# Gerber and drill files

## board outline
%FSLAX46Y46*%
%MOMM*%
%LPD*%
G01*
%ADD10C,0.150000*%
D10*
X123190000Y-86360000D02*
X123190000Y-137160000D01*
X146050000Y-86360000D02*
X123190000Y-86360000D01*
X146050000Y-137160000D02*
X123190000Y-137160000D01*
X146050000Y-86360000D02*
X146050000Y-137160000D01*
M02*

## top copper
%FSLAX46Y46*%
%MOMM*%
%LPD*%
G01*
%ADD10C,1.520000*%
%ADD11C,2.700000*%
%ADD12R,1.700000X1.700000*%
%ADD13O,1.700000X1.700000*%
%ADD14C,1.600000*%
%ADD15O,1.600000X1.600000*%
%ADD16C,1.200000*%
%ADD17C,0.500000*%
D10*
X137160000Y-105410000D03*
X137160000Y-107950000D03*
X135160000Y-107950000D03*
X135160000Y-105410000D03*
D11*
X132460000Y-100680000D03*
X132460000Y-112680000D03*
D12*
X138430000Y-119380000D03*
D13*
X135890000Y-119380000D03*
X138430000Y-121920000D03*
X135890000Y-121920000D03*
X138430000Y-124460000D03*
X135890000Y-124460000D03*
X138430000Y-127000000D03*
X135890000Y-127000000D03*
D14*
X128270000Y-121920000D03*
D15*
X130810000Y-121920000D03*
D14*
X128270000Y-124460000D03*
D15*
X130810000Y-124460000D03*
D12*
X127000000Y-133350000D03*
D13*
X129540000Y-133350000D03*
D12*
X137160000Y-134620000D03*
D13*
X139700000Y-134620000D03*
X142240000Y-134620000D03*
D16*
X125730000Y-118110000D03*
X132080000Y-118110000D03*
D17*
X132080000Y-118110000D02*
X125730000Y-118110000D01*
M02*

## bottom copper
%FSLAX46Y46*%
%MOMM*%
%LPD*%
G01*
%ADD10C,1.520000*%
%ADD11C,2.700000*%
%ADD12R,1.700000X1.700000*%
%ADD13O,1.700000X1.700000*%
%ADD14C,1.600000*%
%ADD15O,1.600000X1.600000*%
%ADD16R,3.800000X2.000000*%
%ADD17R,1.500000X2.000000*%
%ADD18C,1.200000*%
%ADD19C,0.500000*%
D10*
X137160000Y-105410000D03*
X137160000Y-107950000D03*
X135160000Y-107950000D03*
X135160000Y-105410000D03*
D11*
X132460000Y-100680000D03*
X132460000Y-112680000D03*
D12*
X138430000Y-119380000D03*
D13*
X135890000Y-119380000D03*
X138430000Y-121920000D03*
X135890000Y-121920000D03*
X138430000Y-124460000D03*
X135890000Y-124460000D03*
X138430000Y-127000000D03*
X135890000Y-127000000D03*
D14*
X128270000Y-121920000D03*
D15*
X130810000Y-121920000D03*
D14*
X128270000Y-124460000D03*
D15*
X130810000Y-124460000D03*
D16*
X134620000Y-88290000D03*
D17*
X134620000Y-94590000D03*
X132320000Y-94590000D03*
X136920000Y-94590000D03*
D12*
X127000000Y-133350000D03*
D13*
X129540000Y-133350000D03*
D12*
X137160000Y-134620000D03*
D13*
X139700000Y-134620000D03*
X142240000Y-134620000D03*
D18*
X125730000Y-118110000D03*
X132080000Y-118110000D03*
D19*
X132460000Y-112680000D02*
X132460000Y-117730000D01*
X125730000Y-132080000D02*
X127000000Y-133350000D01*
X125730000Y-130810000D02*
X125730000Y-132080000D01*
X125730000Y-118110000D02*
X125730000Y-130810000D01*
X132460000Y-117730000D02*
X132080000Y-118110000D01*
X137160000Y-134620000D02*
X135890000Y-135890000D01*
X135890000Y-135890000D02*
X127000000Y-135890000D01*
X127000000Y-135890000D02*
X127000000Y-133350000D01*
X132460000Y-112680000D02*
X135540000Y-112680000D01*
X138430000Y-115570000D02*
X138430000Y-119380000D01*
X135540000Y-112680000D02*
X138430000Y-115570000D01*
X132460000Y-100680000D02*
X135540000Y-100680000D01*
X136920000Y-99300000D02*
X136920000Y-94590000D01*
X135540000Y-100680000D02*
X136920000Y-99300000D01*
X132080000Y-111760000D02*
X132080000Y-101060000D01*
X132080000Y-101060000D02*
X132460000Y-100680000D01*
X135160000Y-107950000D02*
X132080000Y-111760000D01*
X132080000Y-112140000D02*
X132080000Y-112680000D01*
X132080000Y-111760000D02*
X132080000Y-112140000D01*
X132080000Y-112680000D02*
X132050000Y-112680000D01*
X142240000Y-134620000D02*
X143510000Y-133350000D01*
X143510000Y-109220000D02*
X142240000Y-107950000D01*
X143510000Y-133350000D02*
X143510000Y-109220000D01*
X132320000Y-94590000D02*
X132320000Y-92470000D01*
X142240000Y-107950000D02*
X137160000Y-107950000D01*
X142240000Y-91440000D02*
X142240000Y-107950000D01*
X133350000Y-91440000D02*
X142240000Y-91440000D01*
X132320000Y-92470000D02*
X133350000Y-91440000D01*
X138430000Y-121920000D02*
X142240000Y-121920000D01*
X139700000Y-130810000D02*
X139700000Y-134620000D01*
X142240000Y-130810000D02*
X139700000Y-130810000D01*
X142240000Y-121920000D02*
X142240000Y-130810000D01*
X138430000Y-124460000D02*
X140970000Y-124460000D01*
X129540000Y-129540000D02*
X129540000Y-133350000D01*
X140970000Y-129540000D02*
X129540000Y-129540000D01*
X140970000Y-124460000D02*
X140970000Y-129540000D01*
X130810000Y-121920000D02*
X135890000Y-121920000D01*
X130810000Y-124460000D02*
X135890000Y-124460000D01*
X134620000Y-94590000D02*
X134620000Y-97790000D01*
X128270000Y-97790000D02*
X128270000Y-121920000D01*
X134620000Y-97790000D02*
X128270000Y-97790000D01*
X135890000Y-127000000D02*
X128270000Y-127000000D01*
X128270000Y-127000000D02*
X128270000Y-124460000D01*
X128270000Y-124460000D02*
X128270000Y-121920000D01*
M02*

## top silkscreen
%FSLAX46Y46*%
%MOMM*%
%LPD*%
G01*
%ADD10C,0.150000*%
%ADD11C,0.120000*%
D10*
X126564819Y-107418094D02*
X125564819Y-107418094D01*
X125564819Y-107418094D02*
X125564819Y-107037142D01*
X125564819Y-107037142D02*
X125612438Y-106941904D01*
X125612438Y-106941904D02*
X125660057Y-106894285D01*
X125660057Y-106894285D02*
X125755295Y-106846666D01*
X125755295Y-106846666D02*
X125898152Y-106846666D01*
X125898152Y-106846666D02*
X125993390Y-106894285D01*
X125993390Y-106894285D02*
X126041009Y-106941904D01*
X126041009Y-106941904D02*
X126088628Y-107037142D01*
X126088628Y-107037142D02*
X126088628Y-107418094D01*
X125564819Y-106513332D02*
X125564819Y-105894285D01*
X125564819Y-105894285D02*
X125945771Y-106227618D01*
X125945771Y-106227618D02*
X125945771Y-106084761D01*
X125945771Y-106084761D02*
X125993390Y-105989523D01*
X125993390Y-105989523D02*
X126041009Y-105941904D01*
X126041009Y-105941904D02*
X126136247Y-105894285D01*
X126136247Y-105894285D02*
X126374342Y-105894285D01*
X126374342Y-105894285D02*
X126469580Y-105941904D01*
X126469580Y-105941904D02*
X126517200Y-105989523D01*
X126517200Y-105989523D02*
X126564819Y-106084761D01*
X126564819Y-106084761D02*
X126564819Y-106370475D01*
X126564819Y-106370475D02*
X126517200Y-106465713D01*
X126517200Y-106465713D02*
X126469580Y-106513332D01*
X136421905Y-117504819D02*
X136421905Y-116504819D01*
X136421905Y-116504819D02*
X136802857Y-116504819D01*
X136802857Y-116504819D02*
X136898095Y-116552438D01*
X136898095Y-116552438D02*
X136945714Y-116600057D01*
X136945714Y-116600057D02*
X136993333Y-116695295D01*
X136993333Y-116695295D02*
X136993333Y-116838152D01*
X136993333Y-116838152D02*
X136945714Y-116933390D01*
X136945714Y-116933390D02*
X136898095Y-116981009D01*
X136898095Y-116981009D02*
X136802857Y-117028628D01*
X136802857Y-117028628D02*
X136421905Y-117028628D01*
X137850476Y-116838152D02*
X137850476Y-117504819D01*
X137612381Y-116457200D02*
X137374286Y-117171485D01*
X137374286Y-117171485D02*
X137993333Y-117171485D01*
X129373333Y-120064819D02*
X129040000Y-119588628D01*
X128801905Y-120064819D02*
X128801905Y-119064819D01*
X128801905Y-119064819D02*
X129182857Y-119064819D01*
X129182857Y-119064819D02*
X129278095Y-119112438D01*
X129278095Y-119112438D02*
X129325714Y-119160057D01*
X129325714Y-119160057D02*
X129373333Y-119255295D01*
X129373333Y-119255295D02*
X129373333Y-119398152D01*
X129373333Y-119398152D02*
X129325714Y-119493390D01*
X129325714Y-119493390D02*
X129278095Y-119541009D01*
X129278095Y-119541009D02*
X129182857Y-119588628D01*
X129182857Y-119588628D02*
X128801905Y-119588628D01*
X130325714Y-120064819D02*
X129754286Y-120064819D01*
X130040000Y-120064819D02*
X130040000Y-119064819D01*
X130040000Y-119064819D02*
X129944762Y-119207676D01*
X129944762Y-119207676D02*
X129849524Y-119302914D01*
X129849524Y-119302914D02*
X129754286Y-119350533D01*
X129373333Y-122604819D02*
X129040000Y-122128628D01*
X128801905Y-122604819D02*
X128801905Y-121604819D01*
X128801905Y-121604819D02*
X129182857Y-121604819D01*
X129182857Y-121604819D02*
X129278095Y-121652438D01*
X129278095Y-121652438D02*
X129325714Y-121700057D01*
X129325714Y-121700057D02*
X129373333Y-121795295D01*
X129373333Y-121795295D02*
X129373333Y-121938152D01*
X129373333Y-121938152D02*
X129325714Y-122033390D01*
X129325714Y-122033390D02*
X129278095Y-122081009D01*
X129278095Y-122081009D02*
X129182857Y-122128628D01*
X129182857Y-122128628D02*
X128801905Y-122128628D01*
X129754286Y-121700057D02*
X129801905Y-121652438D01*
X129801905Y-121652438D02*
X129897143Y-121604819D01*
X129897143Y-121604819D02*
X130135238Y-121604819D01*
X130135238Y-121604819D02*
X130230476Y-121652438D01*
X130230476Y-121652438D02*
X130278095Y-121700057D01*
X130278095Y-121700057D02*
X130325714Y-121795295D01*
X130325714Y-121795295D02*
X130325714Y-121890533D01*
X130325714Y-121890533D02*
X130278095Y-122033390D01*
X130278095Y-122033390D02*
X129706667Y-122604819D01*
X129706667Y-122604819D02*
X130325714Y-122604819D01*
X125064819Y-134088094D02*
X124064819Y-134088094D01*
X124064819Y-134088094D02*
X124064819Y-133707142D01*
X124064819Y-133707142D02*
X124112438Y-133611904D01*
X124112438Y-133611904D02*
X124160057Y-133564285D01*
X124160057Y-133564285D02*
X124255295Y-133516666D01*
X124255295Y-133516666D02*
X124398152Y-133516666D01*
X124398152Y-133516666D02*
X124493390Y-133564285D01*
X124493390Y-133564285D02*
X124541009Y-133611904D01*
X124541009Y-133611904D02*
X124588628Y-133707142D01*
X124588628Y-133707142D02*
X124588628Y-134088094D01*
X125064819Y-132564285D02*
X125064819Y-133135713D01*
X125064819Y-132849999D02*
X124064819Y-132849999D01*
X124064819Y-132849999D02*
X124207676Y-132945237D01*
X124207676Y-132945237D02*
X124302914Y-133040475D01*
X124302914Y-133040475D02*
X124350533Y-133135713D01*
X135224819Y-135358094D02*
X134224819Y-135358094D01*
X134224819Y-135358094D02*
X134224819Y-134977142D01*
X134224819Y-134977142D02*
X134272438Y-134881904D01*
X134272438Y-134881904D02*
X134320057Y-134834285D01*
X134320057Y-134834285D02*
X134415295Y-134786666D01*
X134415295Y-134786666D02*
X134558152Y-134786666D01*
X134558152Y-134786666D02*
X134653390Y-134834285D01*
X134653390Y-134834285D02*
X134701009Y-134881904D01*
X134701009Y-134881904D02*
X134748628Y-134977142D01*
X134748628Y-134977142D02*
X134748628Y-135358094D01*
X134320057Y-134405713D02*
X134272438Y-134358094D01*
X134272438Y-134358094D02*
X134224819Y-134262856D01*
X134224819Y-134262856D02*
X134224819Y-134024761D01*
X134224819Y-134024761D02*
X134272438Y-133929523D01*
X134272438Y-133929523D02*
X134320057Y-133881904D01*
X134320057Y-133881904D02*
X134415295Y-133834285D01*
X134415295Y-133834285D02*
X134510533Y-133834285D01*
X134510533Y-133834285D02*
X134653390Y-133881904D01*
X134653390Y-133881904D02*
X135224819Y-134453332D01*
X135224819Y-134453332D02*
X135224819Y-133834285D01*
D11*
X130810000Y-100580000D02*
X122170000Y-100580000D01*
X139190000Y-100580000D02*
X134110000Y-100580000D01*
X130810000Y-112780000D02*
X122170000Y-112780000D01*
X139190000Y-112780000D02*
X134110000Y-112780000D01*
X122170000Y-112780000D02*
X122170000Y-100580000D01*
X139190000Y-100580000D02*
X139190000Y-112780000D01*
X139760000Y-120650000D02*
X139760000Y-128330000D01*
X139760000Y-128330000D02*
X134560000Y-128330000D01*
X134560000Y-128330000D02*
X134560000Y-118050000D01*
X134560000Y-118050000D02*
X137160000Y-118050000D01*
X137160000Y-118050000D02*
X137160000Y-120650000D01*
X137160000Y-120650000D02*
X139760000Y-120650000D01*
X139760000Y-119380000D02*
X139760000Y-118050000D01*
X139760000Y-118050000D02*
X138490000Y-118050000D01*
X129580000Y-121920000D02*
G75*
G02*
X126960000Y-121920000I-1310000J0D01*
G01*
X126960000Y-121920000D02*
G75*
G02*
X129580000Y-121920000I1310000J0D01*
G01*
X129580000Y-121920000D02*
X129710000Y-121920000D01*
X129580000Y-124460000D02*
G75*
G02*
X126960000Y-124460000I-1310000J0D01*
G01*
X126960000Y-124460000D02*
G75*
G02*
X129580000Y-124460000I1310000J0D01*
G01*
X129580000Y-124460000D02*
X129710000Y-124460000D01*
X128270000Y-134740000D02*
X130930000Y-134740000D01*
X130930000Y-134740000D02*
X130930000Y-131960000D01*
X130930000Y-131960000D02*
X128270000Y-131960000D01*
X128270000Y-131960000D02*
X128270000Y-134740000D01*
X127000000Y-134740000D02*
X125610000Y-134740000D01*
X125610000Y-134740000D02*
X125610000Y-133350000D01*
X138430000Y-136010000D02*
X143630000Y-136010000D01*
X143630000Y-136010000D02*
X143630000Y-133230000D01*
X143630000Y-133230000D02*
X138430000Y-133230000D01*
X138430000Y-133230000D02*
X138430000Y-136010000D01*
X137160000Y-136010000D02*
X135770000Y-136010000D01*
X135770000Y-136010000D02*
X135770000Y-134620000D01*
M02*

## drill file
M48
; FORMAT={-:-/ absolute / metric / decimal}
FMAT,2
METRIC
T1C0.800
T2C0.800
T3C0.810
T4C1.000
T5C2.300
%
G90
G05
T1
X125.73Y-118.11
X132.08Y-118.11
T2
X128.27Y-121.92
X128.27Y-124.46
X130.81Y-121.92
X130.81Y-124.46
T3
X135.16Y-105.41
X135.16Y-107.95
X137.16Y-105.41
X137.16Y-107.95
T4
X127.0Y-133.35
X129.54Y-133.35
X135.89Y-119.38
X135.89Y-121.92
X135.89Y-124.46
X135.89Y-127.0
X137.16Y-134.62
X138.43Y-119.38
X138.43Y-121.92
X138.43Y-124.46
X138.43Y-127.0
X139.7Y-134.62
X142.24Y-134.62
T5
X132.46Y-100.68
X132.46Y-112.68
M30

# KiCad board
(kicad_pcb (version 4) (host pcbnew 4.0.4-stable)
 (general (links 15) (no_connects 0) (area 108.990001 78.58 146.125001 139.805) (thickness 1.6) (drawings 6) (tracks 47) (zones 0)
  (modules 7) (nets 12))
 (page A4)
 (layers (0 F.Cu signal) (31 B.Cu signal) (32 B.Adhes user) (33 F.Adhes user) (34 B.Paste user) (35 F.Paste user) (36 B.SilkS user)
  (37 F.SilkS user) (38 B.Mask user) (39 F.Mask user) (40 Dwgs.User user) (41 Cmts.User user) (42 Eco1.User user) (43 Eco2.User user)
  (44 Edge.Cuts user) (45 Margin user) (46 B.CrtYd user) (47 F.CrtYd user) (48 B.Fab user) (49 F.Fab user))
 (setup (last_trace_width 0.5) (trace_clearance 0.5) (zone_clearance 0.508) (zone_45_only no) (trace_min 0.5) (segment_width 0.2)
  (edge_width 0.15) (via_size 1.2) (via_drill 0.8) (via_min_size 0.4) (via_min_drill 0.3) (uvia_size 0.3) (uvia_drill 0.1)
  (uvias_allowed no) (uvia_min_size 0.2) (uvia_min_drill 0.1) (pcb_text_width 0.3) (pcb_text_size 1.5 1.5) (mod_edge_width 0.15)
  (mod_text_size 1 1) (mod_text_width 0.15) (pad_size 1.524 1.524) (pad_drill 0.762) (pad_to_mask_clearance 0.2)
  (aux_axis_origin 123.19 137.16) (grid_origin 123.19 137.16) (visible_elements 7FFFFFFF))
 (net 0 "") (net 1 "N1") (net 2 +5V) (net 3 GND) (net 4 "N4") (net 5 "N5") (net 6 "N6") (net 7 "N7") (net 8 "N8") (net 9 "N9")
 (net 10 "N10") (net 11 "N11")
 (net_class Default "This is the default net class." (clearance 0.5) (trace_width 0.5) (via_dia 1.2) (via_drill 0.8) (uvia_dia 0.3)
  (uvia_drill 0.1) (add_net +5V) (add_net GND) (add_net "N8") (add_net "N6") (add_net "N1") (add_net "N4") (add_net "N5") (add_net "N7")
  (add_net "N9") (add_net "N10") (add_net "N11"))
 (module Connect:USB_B (layer F.Cu) (at 137.16 107.95 180)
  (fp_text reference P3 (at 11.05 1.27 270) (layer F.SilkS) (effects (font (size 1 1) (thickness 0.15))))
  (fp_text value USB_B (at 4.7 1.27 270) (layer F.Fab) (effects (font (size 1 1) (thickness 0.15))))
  (fp_line (start 6.35 7.37) (end 14.99 7.37) (layer F.SilkS) (width 0.12))
  (fp_line (start -2.03 7.37) (end 3.05 7.37) (layer F.SilkS) (width 0.12))
  (fp_line (start 6.35 -4.83) (end 14.99 -4.83) (layer F.SilkS) (width 0.12))
  (fp_line (start -2.03 -4.83) (end 3.05 -4.83) (layer F.SilkS) (width 0.12))
  (fp_line (start 14.99 -4.83) (end 14.99 7.37) (layer F.SilkS) (width 0.12))
  (fp_line (start -2.03 7.37) (end -2.03 -4.83) (layer F.SilkS) (width 0.12))
  (pad 2 thru_hole circle (at 0 2.54 90) (size 1.52 1.52) (drill 0.81) (layers *.Cu *.Mask) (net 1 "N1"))
  (pad 1 thru_hole circle (at 0 0 90) (size 1.52 1.52) (drill 0.81) (layers *.Cu *.Mask) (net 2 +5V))
  (pad 4 thru_hole circle (at 2 0 90) (size 1.52 1.52) (drill 0.81) (layers *.Cu *.Mask) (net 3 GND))
  (pad 3 thru_hole circle (at 2 2.54 90) (size 1.52 1.52) (drill 0.81) (layers *.Cu *.Mask) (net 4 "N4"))
  (pad 5 thru_hole circle (at 4.7 7.27 90) (size 2.7 2.7) (drill 2.3) (layers *.Cu *.Mask) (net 3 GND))
  (pad 5 thru_hole circle (at 4.7 -4.73 90) (size 2.7 2.7) (drill 2.3) (layers *.Cu *.Mask) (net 3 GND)))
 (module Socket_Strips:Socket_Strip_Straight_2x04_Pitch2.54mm (layer F.Cu) (at 138.43 119.38)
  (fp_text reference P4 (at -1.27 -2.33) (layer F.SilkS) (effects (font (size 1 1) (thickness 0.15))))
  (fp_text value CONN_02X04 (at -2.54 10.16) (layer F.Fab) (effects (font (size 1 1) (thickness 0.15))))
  (fp_line (start 1.33 1.27) (end 1.33 8.95) (layer F.SilkS) (width 0.12))
  (fp_line (start 1.33 8.95) (end -3.87 8.95) (layer F.SilkS) (width 0.12))
  (fp_line (start -3.87 8.95) (end -3.87 -1.33) (layer F.SilkS) (width 0.12))
  (fp_line (start -3.87 -1.33) (end -1.27 -1.33) (layer F.SilkS) (width 0.12))
  (fp_line (start -1.27 -1.33) (end -1.27 1.27) (layer F.SilkS) (width 0.12))
  (fp_line (start -1.27 1.27) (end 1.33 1.27) (layer F.SilkS) (width 0.12))
  (fp_line (start 1.33 0) (end 1.33 -1.33) (layer F.SilkS) (width 0.12))
  (fp_line (start 1.33 -1.33) (end 0.06 -1.33) (layer F.SilkS) (width 0.12))
  (pad 1 thru_hole rect (at 0 0) (size 1.7 1.7) (drill 1) (layers *.Cu *.Mask) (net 3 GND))
  (pad 2 thru_hole oval (at -2.54 0) (size 1.7 1.7) (drill 1) (layers *.Cu *.Mask) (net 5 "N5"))
  (pad 3 thru_hole oval (at 0 2.54) (size 1.7 1.7) (drill 1) (layers *.Cu *.Mask) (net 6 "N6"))
  (pad 4 thru_hole oval (at -2.54 2.54) (size 1.7 1.7) (drill 1) (layers *.Cu *.Mask) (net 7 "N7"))
  (pad 5 thru_hole oval (at 0 5.08) (size 1.7 1.7) (drill 1) (layers *.Cu *.Mask) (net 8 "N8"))
  (pad 6 thru_hole oval (at -2.54 5.08) (size 1.7 1.7) (drill 1) (layers *.Cu *.Mask) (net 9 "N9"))
  (pad 7 thru_hole oval (at 0 7.62) (size 1.7 1.7) (drill 1) (layers *.Cu *.Mask) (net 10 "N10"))
  (pad 8 thru_hole oval (at -2.54 7.62) (size 1.7 1.7) (drill 1) (layers *.Cu *.Mask) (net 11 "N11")))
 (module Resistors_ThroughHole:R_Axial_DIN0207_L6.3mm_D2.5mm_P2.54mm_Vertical (layer F.Cu) (at 128.27 121.92)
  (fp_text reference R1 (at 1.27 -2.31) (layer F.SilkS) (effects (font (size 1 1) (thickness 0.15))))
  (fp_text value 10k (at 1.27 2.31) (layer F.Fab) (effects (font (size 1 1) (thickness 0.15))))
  (fp_circle (center 0 0) (end 1.31 0) (layer F.SilkS) (width 0.12))
  (fp_line (start 1.31 0) (end 1.44 0) (layer F.SilkS) (width 0.12))
  (pad 1 thru_hole circle (at 0 0) (size 1.6 1.6) (drill 0.8) (layers *.Cu *.Mask) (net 11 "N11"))
  (pad 2 thru_hole oval (at 2.54 0) (size 1.6 1.6) (drill 0.8) (layers *.Cu *.Mask) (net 7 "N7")))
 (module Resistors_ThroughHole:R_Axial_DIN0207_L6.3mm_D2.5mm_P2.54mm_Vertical (layer F.Cu) (at 128.27 124.46)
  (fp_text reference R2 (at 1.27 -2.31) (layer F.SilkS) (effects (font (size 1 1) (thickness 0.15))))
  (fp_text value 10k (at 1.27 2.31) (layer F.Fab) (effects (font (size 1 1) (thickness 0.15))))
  (fp_circle (center 0 0) (end 1.31 0) (layer F.SilkS) (width 0.12))
  (fp_line (start 1.31 0) (end 1.44 0) (layer F.SilkS) (width 0.12))
  (pad 1 thru_hole circle (at 0 0) (size 1.6 1.6) (drill 0.8) (layers *.Cu *.Mask) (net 11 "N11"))
  (pad 2 thru_hole oval (at 2.54 0) (size 1.6 1.6) (drill 0.8) (layers *.Cu *.Mask) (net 9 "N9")))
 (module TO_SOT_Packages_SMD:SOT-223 (layer B.Cu) (at 134.62 91.44 90)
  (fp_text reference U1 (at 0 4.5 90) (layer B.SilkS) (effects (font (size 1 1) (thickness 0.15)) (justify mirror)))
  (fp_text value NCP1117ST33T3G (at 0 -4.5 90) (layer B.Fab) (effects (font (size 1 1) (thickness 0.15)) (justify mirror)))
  (pad 4 smd rect (at 3.15 0 90) (size 2 3.8) (layers B.Cu B.Paste B.Mask))
  (pad 2 smd rect (at -3.15 0 90) (size 2 1.5) (layers B.Cu B.Paste B.Mask) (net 11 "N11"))
  (pad 3 smd rect (at -3.15 -2.3 90) (size 2 1.5) (layers B.Cu B.Paste B.Mask) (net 2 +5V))
  (pad 1 smd rect (at -3.15 2.3 90) (size 2 1.5) (layers B.Cu B.Paste B.Mask) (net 3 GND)))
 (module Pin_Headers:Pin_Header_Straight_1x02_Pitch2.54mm (layer F.Cu) (at 127 133.35 90)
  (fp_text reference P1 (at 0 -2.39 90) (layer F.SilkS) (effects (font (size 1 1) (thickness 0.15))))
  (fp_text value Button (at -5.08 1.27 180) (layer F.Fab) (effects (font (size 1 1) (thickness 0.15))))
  (fp_line (start -1.39 1.27) (end -1.39 3.93) (layer F.SilkS) (width 0.12))
  (fp_line (start -1.39 3.93) (end 1.39 3.93) (layer F.SilkS) (width 0.12))
  (fp_line (start 1.39 3.93) (end 1.39 1.27) (layer F.SilkS) (width 0.12))
  (fp_line (start 1.39 1.27) (end -1.39 1.27) (layer F.SilkS) (width 0.12))
  (fp_line (start -1.39 0) (end -1.39 -1.39) (layer F.SilkS) (width 0.12))
  (fp_line (start -1.39 -1.39) (end 0 -1.39) (layer F.SilkS) (width 0.12))
  (pad 1 thru_hole rect (at 0 0 90) (size 1.7 1.7) (drill 1) (layers *.Cu *.Mask) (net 3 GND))
  (pad 2 thru_hole oval (at 0 2.54 90) (size 1.7 1.7) (drill 1) (layers *.Cu *.Mask) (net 8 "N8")))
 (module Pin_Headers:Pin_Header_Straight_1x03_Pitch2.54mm (layer F.Cu) (at 137.16 134.62 90)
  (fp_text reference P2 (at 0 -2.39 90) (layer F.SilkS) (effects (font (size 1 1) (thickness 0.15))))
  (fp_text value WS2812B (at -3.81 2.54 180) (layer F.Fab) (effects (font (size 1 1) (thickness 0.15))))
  (fp_line (start -1.39 1.27) (end -1.39 6.47) (layer F.SilkS) (width 0.12))
  (fp_line (start -1.39 6.47) (end 1.39 6.47) (layer F.SilkS) (width 0.12))
  (fp_line (start 1.39 6.47) (end 1.39 1.27) (layer F.SilkS) (width 0.12))
  (fp_line (start 1.39 1.27) (end -1.39 1.27) (layer F.SilkS) (width 0.12))
  (fp_line (start -1.39 0) (end -1.39 -1.39) (layer F.SilkS) (width 0.12))
  (fp_line (start -1.39 -1.39) (end 0 -1.39) (layer F.SilkS) (width 0.12))
  (pad 1 thru_hole rect (at 0 0 90) (size 1.7 1.7) (drill 1) (layers *.Cu *.Mask) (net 3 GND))
  (pad 2 thru_hole oval (at 0 2.54 90) (size 1.7 1.7) (drill 1) (layers *.Cu *.Mask) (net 6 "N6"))
  (pad 3 thru_hole oval (at 0 5.08 90) (size 1.7 1.7) (drill 1) (layers *.Cu *.Mask) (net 2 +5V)))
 (gr_line (start 123.19 86.36) (end 123.19 137.16) (angle 90) (layer Edge.Cuts) (width 0.15))
 (gr_line (start 146.05 86.36) (end 123.19 86.36) (angle 90) (layer Edge.Cuts) (width 0.15))
 (gr_line (start 146.05 137.16) (end 123.19 137.16) (angle 90) (layer Edge.Cuts) (width 0.15))
 (gr_line (start 146.05 86.36) (end 146.05 137.16) (angle 90) (layer Edge.Cuts) (width 0.15))
 (segment (start 132.46 112.68) (end 132.46 117.73) (width 0.5) (layer B.Cu) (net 3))
 (segment (start 125.73 132.08) (end 127 133.35) (width 0.5) (layer B.Cu) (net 3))
 (segment (start 125.73 130.81) (end 125.73 132.08) (width 0.5) (layer B.Cu) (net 3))
 (segment (start 125.73 118.11) (end 125.73 130.81) (width 0.5) (layer B.Cu) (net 3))
 (via (at 125.73 118.11) (size 1.2) (drill 0.8) (layers F.Cu B.Cu) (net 3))
 (segment (start 132.08 118.11) (end 125.73 118.11) (width 0.5) (layer F.Cu) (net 3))
 (via (at 132.08 118.11) (size 1.2) (drill 0.8) (layers F.Cu B.Cu) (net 3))
 (segment (start 132.46 117.73) (end 132.08 118.11) (width 0.5) (layer B.Cu) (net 3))
 (segment (start 137.16 134.62) (end 135.89 135.89) (width 0.5) (layer B.Cu) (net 3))
 (segment (start 135.89 135.89) (end 127 135.89) (width 0.5) (layer B.Cu) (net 3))
 (segment (start 127 135.89) (end 127 133.35) (width 0.5) (layer B.Cu) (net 3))
 (segment (start 132.46 112.68) (end 135.54 112.68) (width 0.5) (layer B.Cu) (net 3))
 (segment (start 138.43 115.57) (end 138.43 119.38) (width 0.5) (layer B.Cu) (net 3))
 (segment (start 135.54 112.68) (end 138.43 115.57) (width 0.5) (layer B.Cu) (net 3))
 (segment (start 132.46 100.68) (end 135.54 100.68) (width 0.5) (layer B.Cu) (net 3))
 (segment (start 136.92 99.3) (end 136.92 94.59) (width 0.5) (layer B.Cu) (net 3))
 (segment (start 135.54 100.68) (end 136.92 99.3) (width 0.5) (layer B.Cu) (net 3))
 (segment (start 132.08 111.76) (end 132.08 101.06) (width 0.5) (layer B.Cu) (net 3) (status 20))
 (segment (start 132.08 101.06) (end 132.46 100.68) (width 0.5) (layer B.Cu) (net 3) (status 30))
 (segment (start 135.16 107.95) (end 132.08 111.76) (width 0.5) (layer B.Cu) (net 3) (status 10))
 (segment (start 132.08 112.14) (end 132.08 112.68) (width 0.5) (layer B.Cu) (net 3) (status 20))
 (segment (start 132.08 111.76) (end 132.08 112.14) (width 0.5) (layer B.Cu) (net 3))
 (segment (start 132.08 112.68) (end 132.05 112.68) (width 0.5) (layer B.Cu) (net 3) (status 30))
 (segment (start 142.24 134.62) (end 143.51 133.35) (width 0.5) (layer B.Cu) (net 2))
 (segment (start 143.51 109.22) (end 142.24 107.95) (width 0.5) (layer B.Cu) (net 2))
 (segment (start 143.51 133.35) (end 143.51 109.22) (width 0.5) (layer B.Cu) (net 2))
 (segment (start 132.32 94.59) (end 132.32 92.47) (width 0.5) (layer B.Cu) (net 2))
 (segment (start 142.24 107.95) (end 137.16 107.95) (width 0.5) (layer B.Cu) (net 2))
 (segment (start 142.24 91.44) (end 142.24 107.95) (width 0.5) (layer B.Cu) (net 2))
 (segment (start 133.35 91.44) (end 142.24 91.44) (width 0.5) (layer B.Cu) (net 2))
 (segment (start 132.32 92.47) (end 133.35 91.44) (width 0.5) (layer B.Cu) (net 2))
 (segment (start 138.43 121.92) (end 142.24 121.92) (width 0.5) (layer B.Cu) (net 6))
 (segment (start 139.7 130.81) (end 139.7 134.62) (width 0.5) (layer B.Cu) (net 6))
 (segment (start 142.24 130.81) (end 139.7 130.81) (width 0.5) (layer B.Cu) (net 6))
 (segment (start 142.24 121.92) (end 142.24 130.81) (width 0.5) (layer B.Cu) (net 6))
 (segment (start 138.43 124.46) (end 140.97 124.46) (width 0.5) (layer B.Cu) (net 8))
 (segment (start 129.54 129.54) (end 129.54 133.35) (width 0.5) (layer B.Cu) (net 8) (status 20))
 (segment (start 140.97 129.54) (end 129.54 129.54) (width 0.5) (layer B.Cu) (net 8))
 (segment (start 140.97 124.46) (end 140.97 129.54) (width 0.5) (layer B.Cu) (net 8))
 (segment (start 130.81 121.92) (end 135.89 121.92) (width 0.5) (layer B.Cu) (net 7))
 (segment (start 130.81 124.46) (end 135.89 124.46) (width 0.5) (layer B.Cu) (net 9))
 (segment (start 134.62 94.59) (end 134.62 97.79) (width 0.5) (layer B.Cu) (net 11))
 (segment (start 128.27 97.79) (end 128.27 121.92) (width 0.5) (layer B.Cu) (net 11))
 (segment (start 134.62 97.79) (end 128.27 97.79) (width 0.5) (layer B.Cu) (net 11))
 (segment (start 135.89 127) (end 128.27 127) (width 0.5) (layer B.Cu) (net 11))
 (segment (start 128.27 127) (end 128.27 124.46) (width 0.5) (layer B.Cu) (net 11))
 (segment (start 128.27 124.46) (end 128.27 121.92) (width 0.5) (layer B.Cu) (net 11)))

